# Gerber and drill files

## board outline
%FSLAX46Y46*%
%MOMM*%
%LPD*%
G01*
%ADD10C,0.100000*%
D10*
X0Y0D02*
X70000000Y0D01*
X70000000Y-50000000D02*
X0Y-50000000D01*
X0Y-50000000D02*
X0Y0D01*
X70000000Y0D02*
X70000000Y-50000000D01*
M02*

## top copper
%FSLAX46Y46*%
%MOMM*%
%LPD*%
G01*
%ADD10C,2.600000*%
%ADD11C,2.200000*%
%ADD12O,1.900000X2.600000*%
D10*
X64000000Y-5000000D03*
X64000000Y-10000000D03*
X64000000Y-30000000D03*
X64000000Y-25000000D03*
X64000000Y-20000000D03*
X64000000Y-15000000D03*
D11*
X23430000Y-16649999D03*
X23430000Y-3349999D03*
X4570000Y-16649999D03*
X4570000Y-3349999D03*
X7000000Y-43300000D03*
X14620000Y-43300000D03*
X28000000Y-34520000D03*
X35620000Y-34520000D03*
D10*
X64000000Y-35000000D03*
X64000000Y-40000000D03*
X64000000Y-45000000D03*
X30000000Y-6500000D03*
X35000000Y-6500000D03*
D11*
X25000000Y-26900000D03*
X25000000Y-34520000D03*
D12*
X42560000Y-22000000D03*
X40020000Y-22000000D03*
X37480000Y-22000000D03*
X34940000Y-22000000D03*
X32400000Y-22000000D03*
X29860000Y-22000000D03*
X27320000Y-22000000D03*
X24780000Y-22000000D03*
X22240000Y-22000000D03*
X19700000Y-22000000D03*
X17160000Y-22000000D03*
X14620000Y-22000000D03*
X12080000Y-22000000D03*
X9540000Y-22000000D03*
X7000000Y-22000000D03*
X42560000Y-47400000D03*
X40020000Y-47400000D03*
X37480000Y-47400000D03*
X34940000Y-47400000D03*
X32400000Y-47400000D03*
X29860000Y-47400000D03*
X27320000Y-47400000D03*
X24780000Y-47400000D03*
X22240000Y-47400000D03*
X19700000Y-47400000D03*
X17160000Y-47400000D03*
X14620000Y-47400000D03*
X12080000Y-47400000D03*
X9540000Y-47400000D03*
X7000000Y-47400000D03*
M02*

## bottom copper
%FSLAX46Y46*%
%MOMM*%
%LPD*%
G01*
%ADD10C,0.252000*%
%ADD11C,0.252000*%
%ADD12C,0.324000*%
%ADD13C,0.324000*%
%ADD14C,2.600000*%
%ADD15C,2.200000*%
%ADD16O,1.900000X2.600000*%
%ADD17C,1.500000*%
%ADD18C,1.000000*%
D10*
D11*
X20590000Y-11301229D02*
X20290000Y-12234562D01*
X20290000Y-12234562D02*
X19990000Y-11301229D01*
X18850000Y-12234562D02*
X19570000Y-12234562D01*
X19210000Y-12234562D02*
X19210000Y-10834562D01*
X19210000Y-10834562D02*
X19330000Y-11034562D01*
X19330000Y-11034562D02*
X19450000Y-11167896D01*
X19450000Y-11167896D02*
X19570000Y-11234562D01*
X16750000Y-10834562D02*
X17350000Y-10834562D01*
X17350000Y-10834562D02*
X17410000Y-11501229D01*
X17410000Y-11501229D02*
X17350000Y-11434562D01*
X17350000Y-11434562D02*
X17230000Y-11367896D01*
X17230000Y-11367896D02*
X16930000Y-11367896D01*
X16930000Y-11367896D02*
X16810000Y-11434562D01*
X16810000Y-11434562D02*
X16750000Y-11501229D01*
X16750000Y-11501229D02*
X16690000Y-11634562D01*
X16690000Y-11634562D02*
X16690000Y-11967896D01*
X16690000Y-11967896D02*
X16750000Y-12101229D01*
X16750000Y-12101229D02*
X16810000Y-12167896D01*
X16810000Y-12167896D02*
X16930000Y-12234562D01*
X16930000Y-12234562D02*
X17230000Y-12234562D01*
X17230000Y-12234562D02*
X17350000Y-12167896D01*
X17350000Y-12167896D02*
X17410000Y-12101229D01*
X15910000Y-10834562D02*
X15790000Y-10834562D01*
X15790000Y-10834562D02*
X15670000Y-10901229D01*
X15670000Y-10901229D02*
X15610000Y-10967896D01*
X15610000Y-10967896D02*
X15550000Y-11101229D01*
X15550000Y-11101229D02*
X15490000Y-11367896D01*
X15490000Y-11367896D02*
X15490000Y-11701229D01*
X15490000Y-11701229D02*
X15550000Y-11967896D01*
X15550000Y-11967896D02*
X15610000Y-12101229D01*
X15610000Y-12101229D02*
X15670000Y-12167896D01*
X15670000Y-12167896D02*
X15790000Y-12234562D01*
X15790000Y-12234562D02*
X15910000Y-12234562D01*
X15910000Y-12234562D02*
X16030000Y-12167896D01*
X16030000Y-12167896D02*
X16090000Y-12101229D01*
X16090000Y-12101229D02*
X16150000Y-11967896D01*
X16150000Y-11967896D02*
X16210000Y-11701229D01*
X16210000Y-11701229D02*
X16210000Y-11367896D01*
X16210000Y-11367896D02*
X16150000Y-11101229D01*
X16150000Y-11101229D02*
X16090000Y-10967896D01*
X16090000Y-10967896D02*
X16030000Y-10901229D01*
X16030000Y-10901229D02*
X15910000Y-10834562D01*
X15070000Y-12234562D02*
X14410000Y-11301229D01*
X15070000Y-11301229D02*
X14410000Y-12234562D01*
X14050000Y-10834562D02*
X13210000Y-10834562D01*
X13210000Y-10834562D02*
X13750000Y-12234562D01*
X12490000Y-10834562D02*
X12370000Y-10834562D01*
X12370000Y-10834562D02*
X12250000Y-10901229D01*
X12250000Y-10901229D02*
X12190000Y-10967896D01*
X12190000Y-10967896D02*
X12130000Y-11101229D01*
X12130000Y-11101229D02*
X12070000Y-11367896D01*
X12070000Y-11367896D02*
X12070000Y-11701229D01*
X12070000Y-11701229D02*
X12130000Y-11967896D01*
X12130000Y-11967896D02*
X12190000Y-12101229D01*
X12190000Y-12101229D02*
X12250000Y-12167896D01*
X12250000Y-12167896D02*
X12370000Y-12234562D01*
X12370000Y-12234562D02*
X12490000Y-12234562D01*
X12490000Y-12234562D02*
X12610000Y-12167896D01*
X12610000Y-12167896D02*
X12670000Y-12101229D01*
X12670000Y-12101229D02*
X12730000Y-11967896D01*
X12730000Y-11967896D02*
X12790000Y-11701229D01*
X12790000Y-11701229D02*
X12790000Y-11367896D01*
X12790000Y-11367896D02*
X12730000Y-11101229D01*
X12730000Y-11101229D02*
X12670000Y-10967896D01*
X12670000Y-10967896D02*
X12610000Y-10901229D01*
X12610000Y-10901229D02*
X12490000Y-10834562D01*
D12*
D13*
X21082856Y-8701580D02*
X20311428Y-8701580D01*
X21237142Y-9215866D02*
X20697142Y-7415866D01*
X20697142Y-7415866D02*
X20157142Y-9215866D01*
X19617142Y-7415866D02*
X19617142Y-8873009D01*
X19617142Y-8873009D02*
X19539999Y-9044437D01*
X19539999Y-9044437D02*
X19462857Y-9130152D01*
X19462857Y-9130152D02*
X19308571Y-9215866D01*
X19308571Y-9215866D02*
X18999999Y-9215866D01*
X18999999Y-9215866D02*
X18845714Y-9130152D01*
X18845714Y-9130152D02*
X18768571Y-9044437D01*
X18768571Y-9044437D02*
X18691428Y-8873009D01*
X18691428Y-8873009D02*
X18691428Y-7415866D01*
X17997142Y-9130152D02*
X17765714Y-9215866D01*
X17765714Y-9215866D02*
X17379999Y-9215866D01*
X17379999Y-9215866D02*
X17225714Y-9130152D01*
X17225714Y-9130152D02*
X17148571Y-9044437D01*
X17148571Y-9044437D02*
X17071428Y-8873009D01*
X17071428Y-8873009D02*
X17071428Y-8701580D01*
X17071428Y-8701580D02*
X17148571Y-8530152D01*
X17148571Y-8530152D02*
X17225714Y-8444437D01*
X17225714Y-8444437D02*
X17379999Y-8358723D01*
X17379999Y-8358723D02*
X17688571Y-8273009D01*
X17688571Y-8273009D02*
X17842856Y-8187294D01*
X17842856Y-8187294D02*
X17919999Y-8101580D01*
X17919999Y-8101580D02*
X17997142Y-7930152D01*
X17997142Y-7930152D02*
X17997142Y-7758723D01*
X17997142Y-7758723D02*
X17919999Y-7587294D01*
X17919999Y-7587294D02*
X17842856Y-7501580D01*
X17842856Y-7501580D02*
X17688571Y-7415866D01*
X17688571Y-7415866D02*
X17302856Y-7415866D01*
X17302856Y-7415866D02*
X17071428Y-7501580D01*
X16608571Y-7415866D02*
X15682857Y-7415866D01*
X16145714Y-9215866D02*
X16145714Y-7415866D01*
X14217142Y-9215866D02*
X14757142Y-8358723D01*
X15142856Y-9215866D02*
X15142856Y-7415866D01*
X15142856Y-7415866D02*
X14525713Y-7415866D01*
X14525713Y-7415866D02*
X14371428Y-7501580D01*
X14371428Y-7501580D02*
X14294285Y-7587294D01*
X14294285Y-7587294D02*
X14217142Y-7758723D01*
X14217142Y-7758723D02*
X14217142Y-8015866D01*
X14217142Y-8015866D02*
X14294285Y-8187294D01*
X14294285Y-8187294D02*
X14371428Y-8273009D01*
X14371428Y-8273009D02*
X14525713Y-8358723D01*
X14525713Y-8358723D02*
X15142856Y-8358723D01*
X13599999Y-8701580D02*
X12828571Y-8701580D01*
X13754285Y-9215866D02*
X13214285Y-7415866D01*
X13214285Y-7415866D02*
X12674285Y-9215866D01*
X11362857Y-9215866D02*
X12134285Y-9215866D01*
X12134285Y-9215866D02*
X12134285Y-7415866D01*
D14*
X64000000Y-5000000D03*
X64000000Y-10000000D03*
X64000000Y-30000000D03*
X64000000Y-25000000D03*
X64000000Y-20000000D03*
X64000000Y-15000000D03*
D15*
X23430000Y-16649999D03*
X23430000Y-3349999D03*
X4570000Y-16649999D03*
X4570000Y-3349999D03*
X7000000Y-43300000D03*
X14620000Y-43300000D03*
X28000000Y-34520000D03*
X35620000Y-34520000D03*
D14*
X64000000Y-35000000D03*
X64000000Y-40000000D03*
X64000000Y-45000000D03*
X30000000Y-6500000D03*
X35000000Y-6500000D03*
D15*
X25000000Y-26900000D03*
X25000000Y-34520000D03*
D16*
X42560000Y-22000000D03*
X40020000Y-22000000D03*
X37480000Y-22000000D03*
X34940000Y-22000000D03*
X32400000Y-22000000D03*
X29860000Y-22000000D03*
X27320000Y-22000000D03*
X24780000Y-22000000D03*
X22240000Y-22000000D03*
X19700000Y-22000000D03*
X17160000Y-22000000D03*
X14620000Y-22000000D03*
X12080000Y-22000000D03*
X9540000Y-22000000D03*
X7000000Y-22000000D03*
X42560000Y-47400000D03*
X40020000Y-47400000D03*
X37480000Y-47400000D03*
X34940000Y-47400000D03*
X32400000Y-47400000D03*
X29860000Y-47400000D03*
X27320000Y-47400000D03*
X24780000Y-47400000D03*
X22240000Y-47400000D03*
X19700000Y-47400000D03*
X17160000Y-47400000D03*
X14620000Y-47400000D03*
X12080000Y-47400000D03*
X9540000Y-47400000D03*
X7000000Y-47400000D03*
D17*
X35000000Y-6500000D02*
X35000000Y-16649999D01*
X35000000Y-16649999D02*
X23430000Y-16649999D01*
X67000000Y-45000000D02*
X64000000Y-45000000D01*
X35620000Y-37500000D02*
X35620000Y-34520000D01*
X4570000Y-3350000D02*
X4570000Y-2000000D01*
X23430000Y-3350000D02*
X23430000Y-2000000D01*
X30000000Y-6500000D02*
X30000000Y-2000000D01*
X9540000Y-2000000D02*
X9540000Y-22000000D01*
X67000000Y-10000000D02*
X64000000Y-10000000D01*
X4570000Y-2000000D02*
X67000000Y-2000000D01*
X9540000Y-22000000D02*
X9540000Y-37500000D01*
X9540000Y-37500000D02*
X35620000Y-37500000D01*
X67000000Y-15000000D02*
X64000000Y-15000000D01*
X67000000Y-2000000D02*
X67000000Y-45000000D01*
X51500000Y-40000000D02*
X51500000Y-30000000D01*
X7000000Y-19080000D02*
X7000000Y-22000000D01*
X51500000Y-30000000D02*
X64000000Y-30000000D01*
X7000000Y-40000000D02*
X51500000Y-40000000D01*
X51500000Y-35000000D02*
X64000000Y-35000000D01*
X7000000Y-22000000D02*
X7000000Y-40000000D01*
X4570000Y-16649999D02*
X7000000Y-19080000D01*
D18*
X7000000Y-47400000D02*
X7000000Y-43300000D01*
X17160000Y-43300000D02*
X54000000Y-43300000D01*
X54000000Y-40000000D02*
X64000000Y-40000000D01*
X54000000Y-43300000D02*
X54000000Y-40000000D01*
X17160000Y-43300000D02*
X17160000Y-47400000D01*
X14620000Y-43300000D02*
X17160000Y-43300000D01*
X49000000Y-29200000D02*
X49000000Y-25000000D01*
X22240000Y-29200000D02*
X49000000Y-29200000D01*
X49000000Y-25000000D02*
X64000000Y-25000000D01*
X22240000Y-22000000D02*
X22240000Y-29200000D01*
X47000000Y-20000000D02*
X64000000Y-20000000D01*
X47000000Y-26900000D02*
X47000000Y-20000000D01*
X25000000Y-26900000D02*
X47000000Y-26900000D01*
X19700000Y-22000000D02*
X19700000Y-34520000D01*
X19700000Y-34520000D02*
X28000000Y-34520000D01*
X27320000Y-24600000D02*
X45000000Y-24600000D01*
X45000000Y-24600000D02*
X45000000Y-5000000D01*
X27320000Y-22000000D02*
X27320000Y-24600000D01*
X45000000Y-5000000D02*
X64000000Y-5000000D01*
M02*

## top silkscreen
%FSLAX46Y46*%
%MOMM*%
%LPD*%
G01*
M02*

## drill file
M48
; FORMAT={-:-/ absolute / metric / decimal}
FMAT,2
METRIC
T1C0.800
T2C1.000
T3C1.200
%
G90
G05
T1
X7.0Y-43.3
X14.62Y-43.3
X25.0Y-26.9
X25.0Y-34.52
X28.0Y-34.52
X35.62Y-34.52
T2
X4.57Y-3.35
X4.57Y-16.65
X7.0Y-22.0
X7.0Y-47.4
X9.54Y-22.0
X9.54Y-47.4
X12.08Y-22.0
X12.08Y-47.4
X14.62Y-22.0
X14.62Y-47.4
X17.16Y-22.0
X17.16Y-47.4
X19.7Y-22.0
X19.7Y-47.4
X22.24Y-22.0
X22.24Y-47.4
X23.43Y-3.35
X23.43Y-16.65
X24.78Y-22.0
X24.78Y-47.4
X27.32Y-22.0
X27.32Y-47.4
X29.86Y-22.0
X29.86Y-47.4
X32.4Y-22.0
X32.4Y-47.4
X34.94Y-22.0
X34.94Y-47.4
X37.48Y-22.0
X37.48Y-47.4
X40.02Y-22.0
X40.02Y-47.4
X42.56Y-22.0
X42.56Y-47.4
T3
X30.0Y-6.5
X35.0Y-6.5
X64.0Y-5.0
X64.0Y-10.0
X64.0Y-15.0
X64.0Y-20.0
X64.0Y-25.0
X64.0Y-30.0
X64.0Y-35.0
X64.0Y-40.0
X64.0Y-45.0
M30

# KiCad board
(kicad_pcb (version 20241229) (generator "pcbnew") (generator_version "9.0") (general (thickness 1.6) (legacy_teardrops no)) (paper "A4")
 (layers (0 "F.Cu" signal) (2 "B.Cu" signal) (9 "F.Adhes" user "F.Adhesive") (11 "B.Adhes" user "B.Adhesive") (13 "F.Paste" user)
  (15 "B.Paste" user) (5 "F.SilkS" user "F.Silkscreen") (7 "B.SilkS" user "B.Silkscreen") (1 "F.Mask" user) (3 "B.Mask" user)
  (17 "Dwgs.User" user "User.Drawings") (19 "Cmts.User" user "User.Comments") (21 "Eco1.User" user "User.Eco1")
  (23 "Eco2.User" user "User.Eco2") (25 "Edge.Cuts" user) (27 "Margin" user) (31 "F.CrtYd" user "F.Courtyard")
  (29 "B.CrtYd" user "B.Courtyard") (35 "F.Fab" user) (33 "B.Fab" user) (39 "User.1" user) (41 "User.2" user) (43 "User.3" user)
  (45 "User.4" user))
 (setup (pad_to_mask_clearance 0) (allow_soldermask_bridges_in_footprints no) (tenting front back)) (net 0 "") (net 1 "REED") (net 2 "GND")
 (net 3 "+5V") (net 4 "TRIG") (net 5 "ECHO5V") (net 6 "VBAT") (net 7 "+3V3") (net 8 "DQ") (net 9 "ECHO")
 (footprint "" (layer "F.Cu") (at 64 7.5)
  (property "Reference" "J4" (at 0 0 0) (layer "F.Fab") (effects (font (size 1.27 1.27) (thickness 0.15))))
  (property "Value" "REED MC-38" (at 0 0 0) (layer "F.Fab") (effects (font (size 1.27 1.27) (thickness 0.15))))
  (pad "1" thru_hole circle (at 0 -2.5) (size 2.6 2.6) (drill 1.2) (layers "*.Cu" "*.Mask") (remove_unused_layers no) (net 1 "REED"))
  (pad "2" thru_hole circle (at 0 2.5) (size 2.6 2.6) (drill 1.2) (layers "*.Cu" "*.Mask") (remove_unused_layers no) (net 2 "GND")))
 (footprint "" (layer "F.Cu") (at 64 22.5)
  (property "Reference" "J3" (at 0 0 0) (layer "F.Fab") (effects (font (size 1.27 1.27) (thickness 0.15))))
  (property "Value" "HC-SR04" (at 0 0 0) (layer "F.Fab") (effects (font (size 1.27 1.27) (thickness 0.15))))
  (pad "1" thru_hole circle (at 0 7.5) (size 2.6 2.6) (drill 1.2) (layers "*.Cu" "*.Mask") (remove_unused_layers no) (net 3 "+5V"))
  (pad "2" thru_hole circle (at 0 2.5) (size 2.6 2.6) (drill 1.2) (layers "*.Cu" "*.Mask") (remove_unused_layers no) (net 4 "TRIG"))
  (pad "3" thru_hole circle (at 0 -2.5) (size 2.6 2.6) (drill 1.2) (layers "*.Cu" "*.Mask") (remove_unused_layers no) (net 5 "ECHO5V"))
  (pad "4" thru_hole circle (at 0 -7.5) (size 2.6 2.6) (drill 1.2) (layers "*.Cu" "*.Mask") (remove_unused_layers no) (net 2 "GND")))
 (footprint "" (layer "F.Cu") (at 14 10)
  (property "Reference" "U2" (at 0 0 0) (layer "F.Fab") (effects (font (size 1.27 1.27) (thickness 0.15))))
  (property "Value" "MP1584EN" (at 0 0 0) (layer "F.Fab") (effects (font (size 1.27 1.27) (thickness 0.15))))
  (pad "IN+" thru_hole circle (at 9.43 6.649999) (size 2.2 2.2) (drill 1) (layers "*.Cu" "*.Mask") (remove_unused_layers no) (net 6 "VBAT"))
  (pad "IN-" thru_hole circle (at 9.43 -6.650001) (size 2.2 2.2) (drill 1) (layers "*.Cu" "*.Mask") (remove_unused_layers no) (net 2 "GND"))
  (pad "OUT+" thru_hole circle (at -9.43 6.649999) (size 2.2 2.2) (drill 1) (layers "*.Cu" "*.Mask") (remove_unused_layers no) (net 3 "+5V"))
  (pad "OUT-" thru_hole circle (at -9.43 -6.650001) (size 2.2 2.2) (drill 1) (layers "*.Cu" "*.Mask") (remove_unused_layers no)
   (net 2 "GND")))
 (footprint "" (layer "F.Cu") (at 10.809999 43.3)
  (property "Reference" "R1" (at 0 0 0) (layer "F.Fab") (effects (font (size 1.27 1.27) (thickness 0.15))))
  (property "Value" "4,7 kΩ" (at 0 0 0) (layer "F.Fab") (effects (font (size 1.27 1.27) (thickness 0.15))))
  (pad "1" thru_hole circle (at -3.809999 0) (size 2.2 2.2) (drill 0.8) (layers "*.Cu" "*.Mask") (remove_unused_layers no) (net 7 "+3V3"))
  (pad "2" thru_hole circle (at 3.810001 0) (size 2.2 2.2) (drill 0.8) (layers "*.Cu" "*.Mask") (remove_unused_layers no) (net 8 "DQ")))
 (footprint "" (layer "F.Cu") (at 31.81 34.52)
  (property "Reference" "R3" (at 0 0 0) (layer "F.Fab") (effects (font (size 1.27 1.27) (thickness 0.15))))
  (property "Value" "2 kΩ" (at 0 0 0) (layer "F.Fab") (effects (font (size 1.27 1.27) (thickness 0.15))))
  (pad "1" thru_hole circle (at -3.81 0) (size 2.2 2.2) (drill 0.8) (layers "*.Cu" "*.Mask") (remove_unused_layers no) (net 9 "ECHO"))
  (pad "2" thru_hole circle (at 3.81 0) (size 2.2 2.2) (drill 0.8) (layers "*.Cu" "*.Mask") (remove_unused_layers no) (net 2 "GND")))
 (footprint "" (layer "F.Cu") (at 64 40)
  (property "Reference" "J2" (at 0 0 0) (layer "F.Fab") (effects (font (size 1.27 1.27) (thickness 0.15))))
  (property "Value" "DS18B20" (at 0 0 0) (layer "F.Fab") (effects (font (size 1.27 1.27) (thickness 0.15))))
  (pad "1" thru_hole circle (at 0 -5) (size 2.6 2.6) (drill 1.2) (layers "*.Cu" "*.Mask") (remove_unused_layers no) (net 3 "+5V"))
  (pad "2" thru_hole circle (at 0 0) (size 2.6 2.6) (drill 1.2) (layers "*.Cu" "*.Mask") (remove_unused_layers no) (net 8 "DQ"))
  (pad "3" thru_hole circle (at 0 5) (size 2.6 2.6) (drill 1.2) (layers "*.Cu" "*.Mask") (remove_unused_layers no) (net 2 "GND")))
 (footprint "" (layer "F.Cu") (at 32.5 6.5)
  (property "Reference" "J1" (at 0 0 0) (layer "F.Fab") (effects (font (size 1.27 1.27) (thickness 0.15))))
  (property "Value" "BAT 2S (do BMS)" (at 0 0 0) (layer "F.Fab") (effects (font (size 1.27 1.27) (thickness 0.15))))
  (pad "1" thru_hole circle (at -2.5 0) (size 2.6 2.6) (drill 1.2) (layers "*.Cu" "*.Mask") (remove_unused_layers no) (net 2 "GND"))
  (pad "2" thru_hole circle (at 2.5 0) (size 2.6 2.6) (drill 1.2) (layers "*.Cu" "*.Mask") (remove_unused_layers no) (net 6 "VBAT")))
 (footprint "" (layer "F.Cu") (at 25 30.71)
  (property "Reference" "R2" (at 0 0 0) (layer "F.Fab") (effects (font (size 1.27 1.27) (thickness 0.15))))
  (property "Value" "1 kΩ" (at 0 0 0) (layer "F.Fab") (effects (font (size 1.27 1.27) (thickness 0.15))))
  (pad "1" thru_hole circle (at 0 -3.81) (size 2.2 2.2) (drill 0.8) (layers "*.Cu" "*.Mask") (remove_unused_layers no) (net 5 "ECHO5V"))
  (pad "2" thru_hole circle (at 0 3.81) (size 2.2 2.2) (drill 0.8) (layers "*.Cu" "*.Mask") (remove_unused_layers no) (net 9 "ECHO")))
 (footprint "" (layer "F.Cu") (at 24.78 34.7)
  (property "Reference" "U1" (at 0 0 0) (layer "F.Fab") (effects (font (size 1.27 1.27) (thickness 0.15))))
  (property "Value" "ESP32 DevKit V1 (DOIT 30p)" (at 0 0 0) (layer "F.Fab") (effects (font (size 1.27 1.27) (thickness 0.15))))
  (pad "1" thru_hole oval (at 17.78 -12.7) (size 1.9 2.6) (drill 1) (layers "*.Cu" "*.Mask") (remove_unused_layers no)
   (thermal_bridge_angle 45))
  (pad "2" thru_hole oval (at 15.24 -12.7) (size 1.9 2.6) (drill 1) (layers "*.Cu" "*.Mask") (remove_unused_layers no)
   (thermal_bridge_angle 45))
  (pad "3" thru_hole oval (at 12.7 -12.7) (size 1.9 2.6) (drill 1) (layers "*.Cu" "*.Mask") (remove_unused_layers no)
   (thermal_bridge_angle 45))
  (pad "4" thru_hole oval (at 10.16 -12.7) (size 1.9 2.6) (drill 1) (layers "*.Cu" "*.Mask") (remove_unused_layers no)
   (thermal_bridge_angle 45))
  (pad "5" thru_hole oval (at 7.62 -12.7) (size 1.9 2.6) (drill 1) (layers "*.Cu" "*.Mask") (remove_unused_layers no)
   (thermal_bridge_angle 45))
  (pad "6" thru_hole oval (at 5.08 -12.7) (size 1.9 2.6) (drill 1) (layers "*.Cu" "*.Mask") (remove_unused_layers no)
   (thermal_bridge_angle 45))
  (pad "7" thru_hole oval (at 2.54 -12.7) (size 1.9 2.6) (drill 1) (layers "*.Cu" "*.Mask") (remove_unused_layers no) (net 1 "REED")
   (thermal_bridge_angle 45))
  (pad "8" thru_hole oval (at 0 -12.7) (size 1.9 2.6) (drill 1) (layers "*.Cu" "*.Mask") (remove_unused_layers no) (thermal_bridge_angle 45))
  (pad "9" thru_hole oval (at -2.54 -12.7) (size 1.9 2.6) (drill 1) (layers "*.Cu" "*.Mask") (remove_unused_layers no) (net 4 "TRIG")
   (thermal_bridge_angle 45))
  (pad "10" thru_hole oval (at -5.08 -12.7) (size 1.9 2.6) (drill 1) (layers "*.Cu" "*.Mask") (remove_unused_layers no) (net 9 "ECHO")
   (thermal_bridge_angle 45))
  (pad "11" thru_hole oval (at -7.62 -12.7) (size 1.9 2.6) (drill 1) (layers "*.Cu" "*.Mask") (remove_unused_layers no)
   (thermal_bridge_angle 45))
  (pad "12" thru_hole oval (at -10.16 -12.7) (size 1.9 2.6) (drill 1) (layers "*.Cu" "*.Mask") (remove_unused_layers no)
   (thermal_bridge_angle 45))
  (pad "13" thru_hole oval (at -12.7 -12.7) (size 1.9 2.6) (drill 1) (layers "*.Cu" "*.Mask") (remove_unused_layers no)
   (thermal_bridge_angle 45))
  (pad "14" thru_hole oval (at -15.24 -12.7) (size 1.9 2.6) (drill 1) (layers "*.Cu" "*.Mask") (remove_unused_layers no) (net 2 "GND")
   (thermal_bridge_angle 45))
  (pad "15" thru_hole oval (at -17.78 -12.7) (size 1.9 2.6) (drill 1) (layers "*.Cu" "*.Mask") (remove_unused_layers no) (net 3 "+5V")
   (thermal_bridge_angle 45))
  (pad "16" thru_hole oval (at 17.78 12.7) (size 1.9 2.6) (drill 1) (layers "*.Cu" "*.Mask") (remove_unused_layers no)
   (thermal_bridge_angle 45))
  (pad "17" thru_hole oval (at 15.24 12.7) (size 1.9 2.6) (drill 1) (layers "*.Cu" "*.Mask") (remove_unused_layers no)
   (thermal_bridge_angle 45))
  (pad "18" thru_hole oval (at 12.7 12.7) (size 1.9 2.6) (drill 1) (layers "*.Cu" "*.Mask") (remove_unused_layers no)
   (thermal_bridge_angle 45))
  (pad "19" thru_hole oval (at 10.16 12.7) (size 1.9 2.6) (drill 1) (layers "*.Cu" "*.Mask") (remove_unused_layers no)
   (thermal_bridge_angle 45))
  (pad "20" thru_hole oval (at 7.62 12.7) (size 1.9 2.6) (drill 1) (layers "*.Cu" "*.Mask") (remove_unused_layers no)
   (thermal_bridge_angle 45))
  (pad "21" thru_hole oval (at 5.08 12.7) (size 1.9 2.6) (drill 1) (layers "*.Cu" "*.Mask") (remove_unused_layers no)
   (thermal_bridge_angle 45))
  (pad "22" thru_hole oval (at 2.54 12.7) (size 1.9 2.6) (drill 1) (layers "*.Cu" "*.Mask") (remove_unused_layers no)
   (thermal_bridge_angle 45))
  (pad "23" thru_hole oval (at 0 12.7) (size 1.9 2.6) (drill 1) (layers "*.Cu" "*.Mask") (remove_unused_layers no) (thermal_bridge_angle 45))
  (pad "24" thru_hole oval (at -2.54 12.7) (size 1.9 2.6) (drill 1) (layers "*.Cu" "*.Mask") (remove_unused_layers no)
   (thermal_bridge_angle 45))
  (pad "25" thru_hole oval (at -5.08 12.7) (size 1.9 2.6) (drill 1) (layers "*.Cu" "*.Mask") (remove_unused_layers no)
   (thermal_bridge_angle 45))
  (pad "26" thru_hole oval (at -7.62 12.7) (size 1.9 2.6) (drill 1) (layers "*.Cu" "*.Mask") (remove_unused_layers no) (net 8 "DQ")
   (thermal_bridge_angle 45))
  (pad "27" thru_hole oval (at -10.16 12.7) (size 1.9 2.6) (drill 1) (layers "*.Cu" "*.Mask") (remove_unused_layers no)
   (thermal_bridge_angle 45))
  (pad "28" thru_hole oval (at -12.7 12.7) (size 1.9 2.6) (drill 1) (layers "*.Cu" "*.Mask") (remove_unused_layers no)
   (thermal_bridge_angle 45))
  (pad "29" thru_hole oval (at -15.24 12.7) (size 1.9 2.6) (drill 1) (layers "*.Cu" "*.Mask") (remove_unused_layers no)
   (thermal_bridge_angle 45))
  (pad "30" thru_hole oval (at -17.78 12.7) (size 1.9 2.6) (drill 1) (layers "*.Cu" "*.Mask") (remove_unused_layers no) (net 7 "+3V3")
   (thermal_bridge_angle 45)))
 (gr_line (start 0 0) (end 70 0) (stroke (width 0.1) (type default)) (layer "Edge.Cuts"))
 (gr_line (start 70 50) (end 0 50) (stroke (width 0.1) (type default)) (layer "Edge.Cuts"))
 (gr_line (start 0 50) (end 0 0) (stroke (width 0.1) (type default)) (layer "Edge.Cuts"))
 (gr_line (start 70 0) (end 70 50) (stroke (width 0.1) (type default)) (layer "Edge.Cuts"))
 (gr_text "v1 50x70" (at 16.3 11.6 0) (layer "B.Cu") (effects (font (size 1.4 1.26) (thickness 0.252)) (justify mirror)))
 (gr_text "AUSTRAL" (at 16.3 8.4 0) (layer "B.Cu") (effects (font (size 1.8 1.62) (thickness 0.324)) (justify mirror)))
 (segment (start 35 6.5) (end 35 16.649999) (width 1.5) (layer "B.Cu") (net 6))
 (segment (start 35 16.649999) (end 23.43 16.649999) (width 1.5) (layer "B.Cu") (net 6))
 (segment (start 67 45) (end 64 45) (width 1.5) (layer "B.Cu") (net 2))
 (segment (start 35.62 37.5) (end 35.62 34.52) (width 1.5) (layer "B.Cu") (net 2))
 (segment (start 4.57 3.35) (end 4.57 2) (width 1.5) (layer "B.Cu") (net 2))
 (segment (start 23.43 3.35) (end 23.43 2) (width 1.5) (layer "B.Cu") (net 2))
 (segment (start 30 6.5) (end 30 2) (width 1.5) (layer "B.Cu") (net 2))
 (segment (start 9.54 2) (end 9.54 22) (width 1.5) (layer "B.Cu") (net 2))
 (segment (start 67 10) (end 64 10) (width 1.5) (layer "B.Cu") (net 2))
 (segment (start 4.57 2) (end 67 2) (width 1.5) (layer "B.Cu") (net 2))
 (segment (start 9.54 22) (end 9.54 37.5) (width 1.5) (layer "B.Cu") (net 2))
 (segment (start 9.54 37.5) (end 35.62 37.5) (width 1.5) (layer "B.Cu") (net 2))
 (segment (start 67 15) (end 64 15) (width 1.5) (layer "B.Cu") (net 2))
 (segment (start 67 2) (end 67 45) (width 1.5) (layer "B.Cu") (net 2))
 (segment (start 51.5 40) (end 51.5 30) (width 1.5) (layer "B.Cu") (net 3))
 (segment (start 7 19.08) (end 7 22) (width 1.5) (layer "B.Cu") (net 3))
 (segment (start 51.5 30) (end 64 30) (width 1.5) (layer "B.Cu") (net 3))
 (segment (start 7 40) (end 51.5 40) (width 1.5) (layer "B.Cu") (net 3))
 (segment (start 51.5 35) (end 64 35) (width 1.5) (layer "B.Cu") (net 3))
 (segment (start 7 22) (end 7 40) (width 1.5) (layer "B.Cu") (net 3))
 (segment (start 4.57 16.649999) (end 7 19.08) (width 1.5) (layer "B.Cu") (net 3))
 (segment (start 7 47.4) (end 7 43.3) (width 1) (layer "B.Cu") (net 7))
 (segment (start 17.16 43.3) (end 54 43.3) (width 1) (layer "B.Cu") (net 8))
 (segment (start 54 40) (end 64 40) (width 1) (layer "B.Cu") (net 8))
 (segment (start 54 43.3) (end 54 40) (width 1) (layer "B.Cu") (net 8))
 (segment (start 17.16 43.3) (end 17.16 47.4) (width 1) (layer "B.Cu") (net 8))
 (segment (start 14.62 43.3) (end 17.16 43.3) (width 1) (layer "B.Cu") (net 8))
 (segment (start 49 29.2) (end 49 25) (width 1) (layer "B.Cu") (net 4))
 (segment (start 22.24 29.2) (end 49 29.2) (width 1) (layer "B.Cu") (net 4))
 (segment (start 49 25) (end 64 25) (width 1) (layer "B.Cu") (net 4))
 (segment (start 22.24 22) (end 22.24 29.2) (width 1) (layer "B.Cu") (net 4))
 (segment (start 47 20) (end 64 20) (width 1) (layer "B.Cu") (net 5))
 (segment (start 47 26.9) (end 47 20) (width 1) (layer "B.Cu") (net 5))
 (segment (start 25 26.9) (end 47 26.9) (width 1) (layer "B.Cu") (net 5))
 (segment (start 19.7 22) (end 19.7 34.52) (width 1) (layer "B.Cu") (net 9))
 (segment (start 19.7 34.52) (end 28 34.52) (width 1) (layer "B.Cu") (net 9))
 (segment (start 27.32 24.6) (end 45 24.6) (width 1) (layer "B.Cu") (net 1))
 (segment (start 45 24.6) (end 45 5) (width 1) (layer "B.Cu") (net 1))
 (segment (start 27.32 22) (end 27.32 24.6) (width 1) (layer "B.Cu") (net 1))
 (segment (start 45 5) (end 64 5) (width 1) (layer "B.Cu") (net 1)))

